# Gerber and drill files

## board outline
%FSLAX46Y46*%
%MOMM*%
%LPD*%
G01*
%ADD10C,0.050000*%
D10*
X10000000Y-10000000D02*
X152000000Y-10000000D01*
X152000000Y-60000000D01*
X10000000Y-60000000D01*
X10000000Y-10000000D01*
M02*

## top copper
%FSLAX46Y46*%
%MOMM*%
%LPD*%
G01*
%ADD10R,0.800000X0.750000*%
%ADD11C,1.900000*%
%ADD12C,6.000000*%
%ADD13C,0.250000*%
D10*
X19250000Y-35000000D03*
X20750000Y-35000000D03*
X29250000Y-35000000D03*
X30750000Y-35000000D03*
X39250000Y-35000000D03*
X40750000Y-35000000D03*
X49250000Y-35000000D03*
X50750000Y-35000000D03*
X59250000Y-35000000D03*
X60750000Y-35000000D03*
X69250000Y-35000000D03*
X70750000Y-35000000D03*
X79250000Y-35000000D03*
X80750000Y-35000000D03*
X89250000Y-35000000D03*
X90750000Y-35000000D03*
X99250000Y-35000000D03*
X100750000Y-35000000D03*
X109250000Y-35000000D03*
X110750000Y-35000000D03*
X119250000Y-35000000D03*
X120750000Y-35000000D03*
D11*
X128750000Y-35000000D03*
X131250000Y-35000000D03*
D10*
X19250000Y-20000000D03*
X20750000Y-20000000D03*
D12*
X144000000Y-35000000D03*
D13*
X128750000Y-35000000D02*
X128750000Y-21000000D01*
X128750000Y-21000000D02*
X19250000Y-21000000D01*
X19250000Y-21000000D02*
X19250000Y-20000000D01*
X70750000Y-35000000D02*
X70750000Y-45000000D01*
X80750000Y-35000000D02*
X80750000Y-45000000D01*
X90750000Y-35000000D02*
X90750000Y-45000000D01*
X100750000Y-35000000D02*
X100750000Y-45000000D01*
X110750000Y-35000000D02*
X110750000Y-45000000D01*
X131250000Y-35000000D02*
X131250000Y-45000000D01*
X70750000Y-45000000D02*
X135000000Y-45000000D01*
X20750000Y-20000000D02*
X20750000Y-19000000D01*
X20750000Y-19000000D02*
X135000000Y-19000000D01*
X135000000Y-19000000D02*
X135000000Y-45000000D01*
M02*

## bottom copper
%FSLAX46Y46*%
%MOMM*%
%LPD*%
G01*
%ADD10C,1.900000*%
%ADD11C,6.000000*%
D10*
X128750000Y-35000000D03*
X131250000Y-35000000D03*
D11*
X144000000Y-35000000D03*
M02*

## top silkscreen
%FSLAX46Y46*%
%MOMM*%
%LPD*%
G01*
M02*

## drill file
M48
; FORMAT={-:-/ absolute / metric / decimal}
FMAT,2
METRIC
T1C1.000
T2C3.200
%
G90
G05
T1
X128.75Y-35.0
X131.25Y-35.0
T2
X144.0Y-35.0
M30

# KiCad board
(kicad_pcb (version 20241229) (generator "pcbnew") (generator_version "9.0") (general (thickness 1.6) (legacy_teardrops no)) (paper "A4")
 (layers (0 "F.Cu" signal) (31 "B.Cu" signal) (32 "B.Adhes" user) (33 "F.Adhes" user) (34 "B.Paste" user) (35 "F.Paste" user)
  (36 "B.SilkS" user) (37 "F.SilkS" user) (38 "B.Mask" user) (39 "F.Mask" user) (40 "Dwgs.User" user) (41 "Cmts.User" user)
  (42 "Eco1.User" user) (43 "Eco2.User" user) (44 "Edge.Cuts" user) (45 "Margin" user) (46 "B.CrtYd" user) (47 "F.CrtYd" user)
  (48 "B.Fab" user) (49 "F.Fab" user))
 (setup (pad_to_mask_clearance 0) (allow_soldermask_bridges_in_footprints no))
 (gr_rect (start 10 10) (end 152 60) (stroke (width 0.05) (type solid)) (fill none) (layer "Edge.Cuts")) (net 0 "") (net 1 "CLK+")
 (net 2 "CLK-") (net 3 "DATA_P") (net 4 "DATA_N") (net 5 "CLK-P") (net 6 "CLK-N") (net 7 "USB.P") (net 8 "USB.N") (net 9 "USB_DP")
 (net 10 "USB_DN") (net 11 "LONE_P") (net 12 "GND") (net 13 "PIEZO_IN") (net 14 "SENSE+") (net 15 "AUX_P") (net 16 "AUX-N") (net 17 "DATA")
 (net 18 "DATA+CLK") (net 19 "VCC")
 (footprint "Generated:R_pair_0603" (layer "F.Cu") (at 20 35)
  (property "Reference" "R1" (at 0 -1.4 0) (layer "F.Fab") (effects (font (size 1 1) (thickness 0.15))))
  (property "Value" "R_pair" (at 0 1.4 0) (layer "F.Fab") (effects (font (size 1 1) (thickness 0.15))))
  (pad "1" smd rect (at -0.75 0) (size 0.8 0.75) (layers "F.Cu" "F.Paste" "F.Mask") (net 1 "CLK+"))
  (pad "2" smd rect (at 0.75 0) (size 0.8 0.75) (layers "F.Cu" "F.Paste" "F.Mask") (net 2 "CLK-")))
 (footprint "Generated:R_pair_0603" (layer "F.Cu") (at 30 35)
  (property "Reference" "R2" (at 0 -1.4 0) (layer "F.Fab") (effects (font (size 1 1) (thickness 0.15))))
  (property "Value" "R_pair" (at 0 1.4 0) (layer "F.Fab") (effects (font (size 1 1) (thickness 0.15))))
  (pad "1" smd rect (at -0.75 0) (size 0.8 0.75) (layers "F.Cu" "F.Paste" "F.Mask") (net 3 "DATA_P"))
  (pad "2" smd rect (at 0.75 0) (size 0.8 0.75) (layers "F.Cu" "F.Paste" "F.Mask") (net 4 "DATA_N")))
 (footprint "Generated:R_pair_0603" (layer "F.Cu") (at 40 35)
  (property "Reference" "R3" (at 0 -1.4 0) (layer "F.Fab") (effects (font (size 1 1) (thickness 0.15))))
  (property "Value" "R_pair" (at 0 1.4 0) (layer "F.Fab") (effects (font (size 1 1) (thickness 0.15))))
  (pad "1" smd rect (at -0.75 0) (size 0.8 0.75) (layers "F.Cu" "F.Paste" "F.Mask") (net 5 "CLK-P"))
  (pad "2" smd rect (at 0.75 0) (size 0.8 0.75) (layers "F.Cu" "F.Paste" "F.Mask") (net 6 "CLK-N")))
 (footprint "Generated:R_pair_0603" (layer "F.Cu") (at 50 35)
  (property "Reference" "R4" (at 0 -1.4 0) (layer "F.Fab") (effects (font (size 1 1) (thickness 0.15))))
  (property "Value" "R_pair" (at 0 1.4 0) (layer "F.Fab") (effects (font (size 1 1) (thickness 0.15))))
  (pad "1" smd rect (at -0.75 0) (size 0.8 0.75) (layers "F.Cu" "F.Paste" "F.Mask") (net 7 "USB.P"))
  (pad "2" smd rect (at 0.75 0) (size 0.8 0.75) (layers "F.Cu" "F.Paste" "F.Mask") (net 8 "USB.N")))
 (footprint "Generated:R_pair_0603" (layer "F.Cu") (at 60 35)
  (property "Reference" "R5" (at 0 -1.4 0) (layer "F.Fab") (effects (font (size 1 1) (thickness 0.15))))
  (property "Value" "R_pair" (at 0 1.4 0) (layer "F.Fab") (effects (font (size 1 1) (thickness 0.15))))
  (pad "1" smd rect (at -0.75 0) (size 0.8 0.75) (layers "F.Cu" "F.Paste" "F.Mask") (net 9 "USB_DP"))
  (pad "2" smd rect (at 0.75 0) (size 0.8 0.75) (layers "F.Cu" "F.Paste" "F.Mask") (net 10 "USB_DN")))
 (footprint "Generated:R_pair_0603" (layer "F.Cu") (at 70 35)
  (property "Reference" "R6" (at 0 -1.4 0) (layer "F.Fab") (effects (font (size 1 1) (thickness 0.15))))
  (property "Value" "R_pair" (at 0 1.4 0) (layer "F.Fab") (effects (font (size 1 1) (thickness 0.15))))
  (pad "1" smd rect (at -0.75 0) (size 0.8 0.75) (layers "F.Cu" "F.Paste" "F.Mask") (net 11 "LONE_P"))
  (pad "2" smd rect (at 0.75 0) (size 0.8 0.75) (layers "F.Cu" "F.Paste" "F.Mask") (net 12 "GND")))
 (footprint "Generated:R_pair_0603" (layer "F.Cu") (at 80 35)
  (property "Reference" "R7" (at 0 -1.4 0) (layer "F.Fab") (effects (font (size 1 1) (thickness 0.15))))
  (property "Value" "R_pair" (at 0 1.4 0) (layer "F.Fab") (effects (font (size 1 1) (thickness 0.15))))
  (pad "1" smd rect (at -0.75 0) (size 0.8 0.75) (layers "F.Cu" "F.Paste" "F.Mask") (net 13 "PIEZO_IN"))
  (pad "2" smd rect (at 0.75 0) (size 0.8 0.75) (layers "F.Cu" "F.Paste" "F.Mask") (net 12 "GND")))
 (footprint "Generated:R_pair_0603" (layer "F.Cu") (at 90 35)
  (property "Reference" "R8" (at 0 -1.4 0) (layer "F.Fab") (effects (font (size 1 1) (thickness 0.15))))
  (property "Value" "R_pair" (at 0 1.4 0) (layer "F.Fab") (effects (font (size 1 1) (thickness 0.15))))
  (pad "1" smd rect (at -0.75 0) (size 0.8 0.75) (layers "F.Cu" "F.Paste" "F.Mask") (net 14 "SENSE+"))
  (pad "2" smd rect (at 0.75 0) (size 0.8 0.75) (layers "F.Cu" "F.Paste" "F.Mask") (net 12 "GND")))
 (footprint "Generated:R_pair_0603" (layer "F.Cu") (at 100 35)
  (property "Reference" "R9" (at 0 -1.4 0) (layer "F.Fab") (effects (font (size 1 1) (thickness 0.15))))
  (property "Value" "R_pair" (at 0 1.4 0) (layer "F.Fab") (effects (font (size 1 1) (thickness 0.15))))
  (pad "1" smd rect (at -0.75 0) (size 0.8 0.75) (layers "F.Cu" "F.Paste" "F.Mask") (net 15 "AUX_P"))
  (pad "2" smd rect (at 0.75 0) (size 0.8 0.75) (layers "F.Cu" "F.Paste" "F.Mask") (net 12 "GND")))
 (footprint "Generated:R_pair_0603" (layer "F.Cu") (at 110 35)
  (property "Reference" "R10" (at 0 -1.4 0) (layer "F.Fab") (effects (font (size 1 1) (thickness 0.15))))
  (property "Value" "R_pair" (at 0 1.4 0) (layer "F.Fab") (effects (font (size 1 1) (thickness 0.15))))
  (pad "1" smd rect (at -0.75 0) (size 0.8 0.75) (layers "F.Cu" "F.Paste" "F.Mask") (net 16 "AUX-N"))
  (pad "2" smd rect (at 0.75 0) (size 0.8 0.75) (layers "F.Cu" "F.Paste" "F.Mask") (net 12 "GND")))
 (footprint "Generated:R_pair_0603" (layer "F.Cu") (at 120 35)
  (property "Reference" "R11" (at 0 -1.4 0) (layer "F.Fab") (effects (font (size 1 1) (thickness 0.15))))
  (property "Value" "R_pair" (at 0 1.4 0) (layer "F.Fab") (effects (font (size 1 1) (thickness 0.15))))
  (pad "1" smd rect (at -0.75 0) (size 0.8 0.75) (layers "F.Cu" "F.Paste" "F.Mask") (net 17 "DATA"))
  (pad "2" smd rect (at 0.75 0) (size 0.8 0.75) (layers "F.Cu" "F.Paste" "F.Mask") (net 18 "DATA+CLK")))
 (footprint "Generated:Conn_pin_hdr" (layer "F.Cu") (at 130 35)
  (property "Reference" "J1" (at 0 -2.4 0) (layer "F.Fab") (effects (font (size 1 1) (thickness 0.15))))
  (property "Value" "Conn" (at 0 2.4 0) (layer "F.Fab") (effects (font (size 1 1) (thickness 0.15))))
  (pad "1" thru_hole circle (at -1.25 0) (size 1.9 1.9) (drill 1.0) (layers "*.Cu" "*.Mask") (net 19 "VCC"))
  (pad "2" thru_hole circle (at 1.25 0) (size 1.9 1.9) (drill 1.0) (layers "*.Cu" "*.Mask") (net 12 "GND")))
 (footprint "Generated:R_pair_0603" (layer "F.Cu") (at 20 20)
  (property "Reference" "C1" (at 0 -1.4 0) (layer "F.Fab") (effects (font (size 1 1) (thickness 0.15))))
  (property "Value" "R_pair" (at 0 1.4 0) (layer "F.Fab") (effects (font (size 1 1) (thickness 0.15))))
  (pad "1" smd rect (at -0.75 0) (size 0.8 0.75) (layers "F.Cu" "F.Paste" "F.Mask") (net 19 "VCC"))
  (pad "2" smd rect (at 0.75 0) (size 0.8 0.75) (layers "F.Cu" "F.Paste" "F.Mask") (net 12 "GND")))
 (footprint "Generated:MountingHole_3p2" (layer "F.Cu") (at 144 35)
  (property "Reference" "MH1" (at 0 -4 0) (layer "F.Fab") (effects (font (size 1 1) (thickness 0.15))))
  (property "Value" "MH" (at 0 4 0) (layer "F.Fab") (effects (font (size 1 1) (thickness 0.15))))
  (pad "1" thru_hole circle (at 0 0) (size 6 6) (drill 3.2) (layers "*.Cu" "*.Mask")))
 (segment (start 128.75 35) (end 128.75 21) (width 0.25) (layer "F.Cu") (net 19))
 (segment (start 128.75 21) (end 19.25 21) (width 0.25) (layer "F.Cu") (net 19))
 (segment (start 19.25 21) (end 19.25 20) (width 0.25) (layer "F.Cu") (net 19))
 (segment (start 70.75 35) (end 70.75 45) (width 0.25) (layer "F.Cu") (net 12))
 (segment (start 80.75 35) (end 80.75 45) (width 0.25) (layer "F.Cu") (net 12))
 (segment (start 90.75 35) (end 90.75 45) (width 0.25) (layer "F.Cu") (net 12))
 (segment (start 100.75 35) (end 100.75 45) (width 0.25) (layer "F.Cu") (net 12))
 (segment (start 110.75 35) (end 110.75 45) (width 0.25) (layer "F.Cu") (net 12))
 (segment (start 131.25 35) (end 131.25 45) (width 0.25) (layer "F.Cu") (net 12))
 (segment (start 70.75 45) (end 135 45) (width 0.25) (layer "F.Cu") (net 12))
 (segment (start 20.75 20) (end 20.75 19) (width 0.25) (layer "F.Cu") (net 12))
 (segment (start 20.75 19) (end 135 19) (width 0.25) (layer "F.Cu") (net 12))
 (segment (start 135 19) (end 135 45) (width 0.25) (layer "F.Cu") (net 12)))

